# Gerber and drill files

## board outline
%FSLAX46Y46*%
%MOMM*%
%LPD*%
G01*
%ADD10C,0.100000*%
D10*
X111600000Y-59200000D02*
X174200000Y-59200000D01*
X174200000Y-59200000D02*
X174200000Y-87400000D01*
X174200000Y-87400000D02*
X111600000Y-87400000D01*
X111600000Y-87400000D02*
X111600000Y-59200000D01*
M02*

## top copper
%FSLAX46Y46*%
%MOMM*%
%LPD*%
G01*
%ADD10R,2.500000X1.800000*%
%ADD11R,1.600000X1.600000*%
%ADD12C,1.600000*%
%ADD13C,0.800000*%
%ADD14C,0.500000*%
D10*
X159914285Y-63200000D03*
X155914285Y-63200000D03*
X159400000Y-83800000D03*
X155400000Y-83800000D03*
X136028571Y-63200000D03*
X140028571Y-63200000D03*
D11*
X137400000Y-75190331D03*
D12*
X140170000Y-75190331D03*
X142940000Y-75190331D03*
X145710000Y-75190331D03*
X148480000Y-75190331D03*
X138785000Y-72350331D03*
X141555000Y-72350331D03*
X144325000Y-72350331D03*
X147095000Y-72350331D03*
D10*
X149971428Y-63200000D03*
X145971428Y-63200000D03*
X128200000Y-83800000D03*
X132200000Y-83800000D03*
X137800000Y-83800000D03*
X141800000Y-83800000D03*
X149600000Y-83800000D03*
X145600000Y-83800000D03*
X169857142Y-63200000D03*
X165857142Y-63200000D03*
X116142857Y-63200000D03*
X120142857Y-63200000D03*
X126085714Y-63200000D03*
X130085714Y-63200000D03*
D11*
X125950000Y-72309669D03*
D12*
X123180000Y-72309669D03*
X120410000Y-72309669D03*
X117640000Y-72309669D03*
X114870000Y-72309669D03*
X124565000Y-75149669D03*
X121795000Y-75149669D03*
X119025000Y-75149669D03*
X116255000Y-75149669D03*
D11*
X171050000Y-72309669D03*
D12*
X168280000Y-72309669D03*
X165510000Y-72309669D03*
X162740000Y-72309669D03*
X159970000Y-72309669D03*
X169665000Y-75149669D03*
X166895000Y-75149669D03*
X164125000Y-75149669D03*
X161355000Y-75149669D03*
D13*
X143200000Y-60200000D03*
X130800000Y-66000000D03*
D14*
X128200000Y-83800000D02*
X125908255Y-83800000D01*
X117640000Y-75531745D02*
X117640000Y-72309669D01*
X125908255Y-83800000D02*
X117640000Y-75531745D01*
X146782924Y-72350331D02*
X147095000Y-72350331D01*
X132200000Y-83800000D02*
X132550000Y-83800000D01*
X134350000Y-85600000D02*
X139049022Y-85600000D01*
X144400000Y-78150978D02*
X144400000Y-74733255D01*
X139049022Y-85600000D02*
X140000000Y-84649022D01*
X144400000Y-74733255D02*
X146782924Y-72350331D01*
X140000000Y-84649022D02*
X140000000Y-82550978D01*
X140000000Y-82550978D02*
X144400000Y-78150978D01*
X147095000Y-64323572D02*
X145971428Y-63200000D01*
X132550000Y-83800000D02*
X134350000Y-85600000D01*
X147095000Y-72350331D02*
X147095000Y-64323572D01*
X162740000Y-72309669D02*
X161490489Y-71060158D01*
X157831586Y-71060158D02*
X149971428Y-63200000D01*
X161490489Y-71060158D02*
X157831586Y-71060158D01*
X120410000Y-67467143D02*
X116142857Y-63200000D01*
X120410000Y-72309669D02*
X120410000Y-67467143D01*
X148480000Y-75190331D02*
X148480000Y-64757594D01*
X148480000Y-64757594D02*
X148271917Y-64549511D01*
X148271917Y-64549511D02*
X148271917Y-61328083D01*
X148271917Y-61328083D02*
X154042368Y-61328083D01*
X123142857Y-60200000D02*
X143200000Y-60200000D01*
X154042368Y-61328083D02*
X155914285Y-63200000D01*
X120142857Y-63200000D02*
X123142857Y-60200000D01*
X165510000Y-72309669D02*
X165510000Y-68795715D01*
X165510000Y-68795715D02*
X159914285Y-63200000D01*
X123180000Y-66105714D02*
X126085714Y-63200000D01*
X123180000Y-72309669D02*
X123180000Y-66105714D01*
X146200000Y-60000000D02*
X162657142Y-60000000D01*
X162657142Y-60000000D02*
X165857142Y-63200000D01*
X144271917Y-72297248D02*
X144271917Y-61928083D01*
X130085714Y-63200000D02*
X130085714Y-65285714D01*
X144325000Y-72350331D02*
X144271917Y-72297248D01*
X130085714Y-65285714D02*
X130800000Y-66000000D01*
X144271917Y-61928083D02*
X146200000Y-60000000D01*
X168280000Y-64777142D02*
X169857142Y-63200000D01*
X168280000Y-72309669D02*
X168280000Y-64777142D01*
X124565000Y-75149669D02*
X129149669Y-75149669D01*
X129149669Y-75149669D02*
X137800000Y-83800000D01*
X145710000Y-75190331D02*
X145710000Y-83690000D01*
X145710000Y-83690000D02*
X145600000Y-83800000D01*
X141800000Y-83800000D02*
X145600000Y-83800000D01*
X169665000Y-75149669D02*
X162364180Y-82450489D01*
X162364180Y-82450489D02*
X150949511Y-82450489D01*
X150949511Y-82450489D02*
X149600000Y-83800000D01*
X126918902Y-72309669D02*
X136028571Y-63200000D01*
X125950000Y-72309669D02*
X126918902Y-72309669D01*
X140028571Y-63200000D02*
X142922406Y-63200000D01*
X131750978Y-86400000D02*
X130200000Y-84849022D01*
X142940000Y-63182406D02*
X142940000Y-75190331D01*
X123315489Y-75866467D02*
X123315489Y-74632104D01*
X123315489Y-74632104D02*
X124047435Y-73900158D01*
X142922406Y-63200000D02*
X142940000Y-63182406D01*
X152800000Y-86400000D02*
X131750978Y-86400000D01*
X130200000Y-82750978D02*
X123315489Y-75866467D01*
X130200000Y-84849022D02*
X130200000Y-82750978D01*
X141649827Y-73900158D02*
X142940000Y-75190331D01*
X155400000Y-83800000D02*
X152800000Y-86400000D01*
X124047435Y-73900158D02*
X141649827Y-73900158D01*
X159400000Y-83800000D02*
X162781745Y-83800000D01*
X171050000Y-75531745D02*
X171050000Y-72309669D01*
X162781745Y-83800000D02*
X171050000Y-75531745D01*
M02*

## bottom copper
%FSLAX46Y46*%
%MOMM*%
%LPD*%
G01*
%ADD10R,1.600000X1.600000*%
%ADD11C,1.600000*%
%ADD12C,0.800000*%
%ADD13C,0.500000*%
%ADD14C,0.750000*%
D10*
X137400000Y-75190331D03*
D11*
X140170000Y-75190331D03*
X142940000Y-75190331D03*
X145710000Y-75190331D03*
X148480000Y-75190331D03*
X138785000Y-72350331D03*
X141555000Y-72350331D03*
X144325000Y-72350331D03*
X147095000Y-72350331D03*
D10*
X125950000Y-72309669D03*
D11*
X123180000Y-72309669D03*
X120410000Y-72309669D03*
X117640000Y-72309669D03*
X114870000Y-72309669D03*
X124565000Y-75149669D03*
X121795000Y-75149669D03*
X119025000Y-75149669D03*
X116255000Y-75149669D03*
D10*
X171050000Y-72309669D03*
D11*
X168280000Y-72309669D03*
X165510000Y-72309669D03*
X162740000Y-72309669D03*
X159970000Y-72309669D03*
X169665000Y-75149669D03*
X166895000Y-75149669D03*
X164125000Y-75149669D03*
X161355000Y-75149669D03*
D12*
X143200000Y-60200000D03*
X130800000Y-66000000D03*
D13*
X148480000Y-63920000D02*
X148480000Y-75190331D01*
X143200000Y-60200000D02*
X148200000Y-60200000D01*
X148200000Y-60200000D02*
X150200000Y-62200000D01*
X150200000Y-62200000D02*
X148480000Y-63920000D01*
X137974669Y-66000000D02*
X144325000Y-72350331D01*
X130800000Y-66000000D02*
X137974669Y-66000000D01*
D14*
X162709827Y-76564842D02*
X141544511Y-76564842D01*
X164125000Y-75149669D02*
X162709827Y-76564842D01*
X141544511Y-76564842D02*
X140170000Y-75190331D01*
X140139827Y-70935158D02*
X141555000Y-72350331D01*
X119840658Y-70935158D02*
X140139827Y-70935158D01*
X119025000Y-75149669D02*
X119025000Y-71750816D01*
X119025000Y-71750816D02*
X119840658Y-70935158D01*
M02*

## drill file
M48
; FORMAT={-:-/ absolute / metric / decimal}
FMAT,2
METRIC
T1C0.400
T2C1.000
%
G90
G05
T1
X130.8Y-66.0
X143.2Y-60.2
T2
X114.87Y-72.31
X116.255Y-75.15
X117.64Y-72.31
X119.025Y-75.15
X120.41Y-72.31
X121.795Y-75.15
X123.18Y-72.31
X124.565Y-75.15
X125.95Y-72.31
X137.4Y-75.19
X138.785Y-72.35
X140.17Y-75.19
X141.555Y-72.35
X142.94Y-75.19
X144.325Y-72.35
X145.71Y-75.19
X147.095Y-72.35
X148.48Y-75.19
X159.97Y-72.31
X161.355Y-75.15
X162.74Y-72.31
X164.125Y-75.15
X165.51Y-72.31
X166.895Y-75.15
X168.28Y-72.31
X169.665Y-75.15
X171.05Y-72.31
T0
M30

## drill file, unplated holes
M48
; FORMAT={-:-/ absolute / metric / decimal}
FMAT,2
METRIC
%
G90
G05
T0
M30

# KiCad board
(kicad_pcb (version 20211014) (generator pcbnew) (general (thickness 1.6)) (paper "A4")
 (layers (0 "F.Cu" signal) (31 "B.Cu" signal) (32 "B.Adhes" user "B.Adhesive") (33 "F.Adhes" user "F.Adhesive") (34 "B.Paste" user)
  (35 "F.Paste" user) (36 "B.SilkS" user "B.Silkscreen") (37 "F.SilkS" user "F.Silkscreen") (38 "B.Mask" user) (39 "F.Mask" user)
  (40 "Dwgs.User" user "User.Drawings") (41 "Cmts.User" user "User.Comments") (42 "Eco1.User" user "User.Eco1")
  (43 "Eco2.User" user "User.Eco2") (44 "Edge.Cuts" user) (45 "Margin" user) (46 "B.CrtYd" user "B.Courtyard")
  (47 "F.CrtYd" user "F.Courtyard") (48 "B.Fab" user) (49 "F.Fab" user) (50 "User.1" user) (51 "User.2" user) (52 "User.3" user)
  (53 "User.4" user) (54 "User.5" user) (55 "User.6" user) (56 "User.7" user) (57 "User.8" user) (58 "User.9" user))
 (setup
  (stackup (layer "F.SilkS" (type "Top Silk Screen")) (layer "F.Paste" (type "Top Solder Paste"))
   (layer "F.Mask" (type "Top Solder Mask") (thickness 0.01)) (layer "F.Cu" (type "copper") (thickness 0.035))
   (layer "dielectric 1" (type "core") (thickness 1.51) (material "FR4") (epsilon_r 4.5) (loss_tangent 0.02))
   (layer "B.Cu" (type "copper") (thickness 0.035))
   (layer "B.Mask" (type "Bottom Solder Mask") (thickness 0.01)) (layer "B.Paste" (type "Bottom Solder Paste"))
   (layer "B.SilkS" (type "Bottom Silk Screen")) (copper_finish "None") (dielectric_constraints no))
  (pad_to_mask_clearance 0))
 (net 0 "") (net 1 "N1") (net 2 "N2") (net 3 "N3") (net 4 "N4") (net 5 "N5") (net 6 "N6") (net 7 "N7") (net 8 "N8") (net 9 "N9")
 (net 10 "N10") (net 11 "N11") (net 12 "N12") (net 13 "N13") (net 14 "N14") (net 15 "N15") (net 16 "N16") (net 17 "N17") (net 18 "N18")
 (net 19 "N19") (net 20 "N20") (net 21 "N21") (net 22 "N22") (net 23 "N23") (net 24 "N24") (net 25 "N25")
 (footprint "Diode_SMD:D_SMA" (layer "F.Cu") (at 157.914285 63.2 180)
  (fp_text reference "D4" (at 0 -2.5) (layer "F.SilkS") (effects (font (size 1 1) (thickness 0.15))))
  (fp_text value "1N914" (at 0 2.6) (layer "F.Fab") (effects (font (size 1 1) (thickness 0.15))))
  (pad "1" smd rect (at -2 0 180) (size 2.5 1.8) (layers "F.Cu" "F.Paste" "F.Mask") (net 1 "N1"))
  (pad "2" smd rect (at 2 0 180) (size 2.5 1.8) (layers "F.Cu" "F.Paste" "F.Mask") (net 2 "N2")))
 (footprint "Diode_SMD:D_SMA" (layer "F.Cu") (at 157.4 83.8 180)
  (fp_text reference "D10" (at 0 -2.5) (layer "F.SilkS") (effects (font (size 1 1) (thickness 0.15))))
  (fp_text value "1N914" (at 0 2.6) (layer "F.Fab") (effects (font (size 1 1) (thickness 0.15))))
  (pad "1" smd rect (at -2 0 180) (size 2.5 1.8) (layers "F.Cu" "F.Paste" "F.Mask") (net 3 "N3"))
  (pad "2" smd rect (at 2 0 180) (size 2.5 1.8) (layers "F.Cu" "F.Paste" "F.Mask") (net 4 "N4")))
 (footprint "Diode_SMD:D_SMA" (layer "F.Cu") (at 138.028571 63.2)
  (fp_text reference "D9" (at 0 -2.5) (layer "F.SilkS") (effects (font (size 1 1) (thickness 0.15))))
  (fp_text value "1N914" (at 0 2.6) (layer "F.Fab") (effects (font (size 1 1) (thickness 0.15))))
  (pad "1" smd rect (at -2 0) (size 2.5 1.8) (layers "F.Cu" "F.Paste" "F.Mask") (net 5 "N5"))
  (pad "2" smd rect (at 2 0) (size 2.5 1.8) (layers "F.Cu" "F.Paste" "F.Mask") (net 4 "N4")))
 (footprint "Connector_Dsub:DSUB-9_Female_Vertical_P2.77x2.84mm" (layer "F.Cu") (at 137.4 75.190331 180)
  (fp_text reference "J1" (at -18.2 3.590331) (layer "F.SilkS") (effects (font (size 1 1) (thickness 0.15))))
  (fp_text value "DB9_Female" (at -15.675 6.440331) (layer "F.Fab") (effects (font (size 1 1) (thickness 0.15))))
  (pad "1" thru_hole rect (at 0 0 180) (size 1.6 1.6) (drill 1) (layers *.Cu *.Mask) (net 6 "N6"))
  (pad "2" thru_hole circle (at -2.77 0 180) (size 1.6 1.6) (drill 1) (layers *.Cu *.Mask) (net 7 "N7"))
  (pad "3" thru_hole circle (at -5.54 0 180) (size 1.6 1.6) (drill 1) (layers *.Cu *.Mask) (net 4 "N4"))
  (pad "4" thru_hole circle (at -8.31 0 180) (size 1.6 1.6) (drill 1) (layers *.Cu *.Mask) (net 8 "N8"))
  (pad "5" thru_hole circle (at -11.08 0 180) (size 1.6 1.6) (drill 1) (layers *.Cu *.Mask) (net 2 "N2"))
  (pad "6" thru_hole circle (at -1.385 2.84 180) (size 1.6 1.6) (drill 1) (layers *.Cu *.Mask) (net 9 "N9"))
  (pad "7" thru_hole circle (at -4.155 2.84 180) (size 1.6 1.6) (drill 1) (layers *.Cu *.Mask) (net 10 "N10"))
  (pad "8" thru_hole circle (at -6.925 2.84 180) (size 1.6 1.6) (drill 1) (layers *.Cu *.Mask) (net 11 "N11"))
  (pad "9" thru_hole circle (at -9.695 2.84 180) (size 1.6 1.6) (drill 1) (layers *.Cu *.Mask) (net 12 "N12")))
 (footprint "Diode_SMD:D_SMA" (layer "F.Cu") (at 147.971428 63.2 180)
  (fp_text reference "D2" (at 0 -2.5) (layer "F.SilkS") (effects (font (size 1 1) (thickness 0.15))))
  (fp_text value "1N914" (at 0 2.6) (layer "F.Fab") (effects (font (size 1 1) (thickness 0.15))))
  (pad "1" smd rect (at -2 0 180) (size 2.5 1.8) (layers "F.Cu" "F.Paste" "F.Mask") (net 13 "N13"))
  (pad "2" smd rect (at 2 0 180) (size 2.5 1.8) (layers "F.Cu" "F.Paste" "F.Mask") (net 12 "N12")))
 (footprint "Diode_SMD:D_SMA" (layer "F.Cu") (at 130.2 83.8)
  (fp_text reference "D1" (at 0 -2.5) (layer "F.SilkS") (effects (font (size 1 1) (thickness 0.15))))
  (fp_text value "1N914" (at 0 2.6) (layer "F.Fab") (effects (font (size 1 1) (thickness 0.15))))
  (pad "1" smd rect (at -2 0) (size 2.5 1.8) (layers "F.Cu" "F.Paste" "F.Mask") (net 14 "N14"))
  (pad "2" smd rect (at 2 0) (size 2.5 1.8) (layers "F.Cu" "F.Paste" "F.Mask") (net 12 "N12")))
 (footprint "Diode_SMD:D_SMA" (layer "F.Cu") (at 139.8 83.8)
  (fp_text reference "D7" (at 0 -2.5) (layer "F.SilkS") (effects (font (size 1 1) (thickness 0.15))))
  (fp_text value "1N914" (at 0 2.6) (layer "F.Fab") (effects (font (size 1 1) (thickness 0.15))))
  (pad "1" smd rect (at -2 0) (size 2.5 1.8) (layers "F.Cu" "F.Paste" "F.Mask") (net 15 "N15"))
  (pad "2" smd rect (at 2 0) (size 2.5 1.8) (layers "F.Cu" "F.Paste" "F.Mask") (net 8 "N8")))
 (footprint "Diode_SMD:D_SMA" (layer "F.Cu") (at 147.6 83.8 180)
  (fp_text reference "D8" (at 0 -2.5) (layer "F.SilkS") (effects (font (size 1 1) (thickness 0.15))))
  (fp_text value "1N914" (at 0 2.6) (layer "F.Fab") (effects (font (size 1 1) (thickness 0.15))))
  (pad "1" smd rect (at -2 0 180) (size 2.5 1.8) (layers "F.Cu" "F.Paste" "F.Mask") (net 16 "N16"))
  (pad "2" smd rect (at 2 0 180) (size 2.5 1.8) (layers "F.Cu" "F.Paste" "F.Mask") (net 8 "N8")))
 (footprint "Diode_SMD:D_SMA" (layer "F.Cu") (at 167.857142 63.2 180)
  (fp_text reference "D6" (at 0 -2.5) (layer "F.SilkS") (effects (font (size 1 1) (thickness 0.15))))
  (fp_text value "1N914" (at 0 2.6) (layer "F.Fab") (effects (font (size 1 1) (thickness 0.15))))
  (pad "1" smd rect (at -2 0 180) (size 2.5 1.8) (layers "F.Cu" "F.Paste" "F.Mask") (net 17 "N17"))
  (pad "2" smd rect (at 2 0 180) (size 2.5 1.8) (layers "F.Cu" "F.Paste" "F.Mask") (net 11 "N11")))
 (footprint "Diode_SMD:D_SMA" (layer "F.Cu") (at 118.142857 63.2)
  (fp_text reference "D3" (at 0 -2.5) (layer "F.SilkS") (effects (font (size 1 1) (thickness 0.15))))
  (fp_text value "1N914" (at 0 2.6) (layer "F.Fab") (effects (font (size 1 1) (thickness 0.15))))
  (pad "1" smd rect (at -2 0) (size 2.5 1.8) (layers "F.Cu" "F.Paste" "F.Mask") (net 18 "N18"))
  (pad "2" smd rect (at 2 0) (size 2.5 1.8) (layers "F.Cu" "F.Paste" "F.Mask") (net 2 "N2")))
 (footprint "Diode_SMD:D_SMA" (layer "F.Cu") (at 128.085714 63.2)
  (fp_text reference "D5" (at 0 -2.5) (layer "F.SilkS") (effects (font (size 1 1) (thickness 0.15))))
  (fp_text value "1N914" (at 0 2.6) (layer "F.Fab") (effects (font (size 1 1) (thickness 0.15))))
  (pad "1" smd rect (at -2 0) (size 2.5 1.8) (layers "F.Cu" "F.Paste" "F.Mask") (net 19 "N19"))
  (pad "2" smd rect (at 2 0) (size 2.5 1.8) (layers "F.Cu" "F.Paste" "F.Mask") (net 11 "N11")))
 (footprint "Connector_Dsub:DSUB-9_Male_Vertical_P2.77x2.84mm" (layer "B.Cu") (at 125.95 72.309669 180)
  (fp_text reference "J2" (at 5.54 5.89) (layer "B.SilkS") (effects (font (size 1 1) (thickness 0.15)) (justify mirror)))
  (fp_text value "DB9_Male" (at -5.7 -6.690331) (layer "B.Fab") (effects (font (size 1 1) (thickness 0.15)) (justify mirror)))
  (pad "1" thru_hole rect (at 0 0 180) (size 1.6 1.6) (drill 1) (layers *.Cu *.Mask) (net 5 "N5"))
  (pad "2" thru_hole circle (at 2.77 0 180) (size 1.6 1.6) (drill 1) (layers *.Cu *.Mask) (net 19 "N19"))
  (pad "3" thru_hole circle (at 5.54 0 180) (size 1.6 1.6) (drill 1) (layers *.Cu *.Mask) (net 18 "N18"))
  (pad "4" thru_hole circle (at 8.31 0 180) (size 1.6 1.6) (drill 1) (layers *.Cu *.Mask) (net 14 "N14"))
  (pad "5" thru_hole circle (at 11.08 0 180) (size 1.6 1.6) (drill 1) (layers *.Cu *.Mask) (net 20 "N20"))
  (pad "6" thru_hole circle (at 1.385 -2.84 180) (size 1.6 1.6) (drill 1) (layers *.Cu *.Mask) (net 15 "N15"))
  (pad "7" thru_hole circle (at 4.155 -2.84 180) (size 1.6 1.6) (drill 1) (layers *.Cu *.Mask) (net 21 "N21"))
  (pad "8" thru_hole circle (at 6.925 -2.84 180) (size 1.6 1.6) (drill 1) (layers *.Cu *.Mask) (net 10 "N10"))
  (pad "9" thru_hole circle (at 9.695 -2.84 180) (size 1.6 1.6) (drill 1) (layers *.Cu *.Mask) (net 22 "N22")))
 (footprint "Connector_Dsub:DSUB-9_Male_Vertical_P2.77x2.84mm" (layer "B.Cu") (at 171.05 72.309669 180)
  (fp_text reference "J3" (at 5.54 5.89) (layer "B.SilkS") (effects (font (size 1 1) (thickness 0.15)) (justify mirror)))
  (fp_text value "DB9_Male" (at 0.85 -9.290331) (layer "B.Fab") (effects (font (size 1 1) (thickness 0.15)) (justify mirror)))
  (pad "1" thru_hole rect (at 0 0 180) (size 1.6 1.6) (drill 1) (layers *.Cu *.Mask) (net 3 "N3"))
  (pad "2" thru_hole circle (at 2.77 0 180) (size 1.6 1.6) (drill 1) (layers *.Cu *.Mask) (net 17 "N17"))
  (pad "3" thru_hole circle (at 5.54 0 180) (size 1.6 1.6) (drill 1) (layers *.Cu *.Mask) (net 1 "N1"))
  (pad "4" thru_hole circle (at 8.31 0 180) (size 1.6 1.6) (drill 1) (layers *.Cu *.Mask) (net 13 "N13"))
  (pad "5" thru_hole circle (at 11.08 0 180) (size 1.6 1.6) (drill 1) (layers *.Cu *.Mask) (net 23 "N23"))
  (pad "6" thru_hole circle (at 1.385 -2.84 180) (size 1.6 1.6) (drill 1) (layers *.Cu *.Mask) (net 16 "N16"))
  (pad "7" thru_hole circle (at 4.155 -2.84 180) (size 1.6 1.6) (drill 1) (layers *.Cu *.Mask) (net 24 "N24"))
  (pad "8" thru_hole circle (at 6.925 -2.84 180) (size 1.6 1.6) (drill 1) (layers *.Cu *.Mask) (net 7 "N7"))
  (pad "9" thru_hole circle (at 9.695 -2.84 180) (size 1.6 1.6) (drill 1) (layers *.Cu *.Mask) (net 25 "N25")))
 (gr_rect (start 111.6 59.2) (end 174.2 87.4) (layer "Edge.Cuts") (width 0.1) (fill none))
 (segment (start 128.2 83.8) (end 125.908255 83.8) (width 0.5) (layer "F.Cu") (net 14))
 (segment (start 117.64 75.531745) (end 117.64 72.309669) (width 0.5) (layer "F.Cu") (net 14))
 (segment (start 125.908255 83.8) (end 117.64 75.531745) (width 0.5) (layer "F.Cu") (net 14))
 (segment (start 146.782924 72.350331) (end 147.095 72.350331) (width 0.5) (layer "F.Cu") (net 12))
 (segment (start 132.2 83.8) (end 132.55 83.8) (width 0.5) (layer "F.Cu") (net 12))
 (segment (start 134.35 85.6) (end 139.049022 85.6) (width 0.5) (layer "F.Cu") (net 12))
 (segment (start 144.4 78.150978) (end 144.4 74.733255) (width 0.5) (layer "F.Cu") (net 12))
 (segment (start 139.049022 85.6) (end 140 84.649022) (width 0.5) (layer "F.Cu") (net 12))
 (segment (start 144.4 74.733255) (end 146.782924 72.350331) (width 0.5) (layer "F.Cu") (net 12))
 (segment (start 140 84.649022) (end 140 82.550978) (width 0.5) (layer "F.Cu") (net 12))
 (segment (start 140 82.550978) (end 144.4 78.150978) (width 0.5) (layer "F.Cu") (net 12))
 (segment (start 147.095 64.323572) (end 145.971428 63.2) (width 0.5) (layer "F.Cu") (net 12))
 (segment (start 132.55 83.8) (end 134.35 85.6) (width 0.5) (layer "F.Cu") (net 12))
 (segment (start 147.095 72.350331) (end 147.095 64.323572) (width 0.5) (layer "F.Cu") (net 12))
 (segment (start 162.74 72.309669) (end 161.490489 71.060158) (width 0.5) (layer "F.Cu") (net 13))
 (segment (start 157.831586 71.060158) (end 149.971428 63.2) (width 0.5) (layer "F.Cu") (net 13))
 (segment (start 161.490489 71.060158) (end 157.831586 71.060158) (width 0.5) (layer "F.Cu") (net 13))
 (segment (start 120.41 67.467143) (end 116.142857 63.2) (width 0.5) (layer "F.Cu") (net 18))
 (segment (start 120.41 72.309669) (end 120.41 67.467143) (width 0.5) (layer "F.Cu") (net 18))
 (segment (start 148.48 75.190331) (end 148.48 64.757594) (width 0.5) (layer "F.Cu") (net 2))
 (segment (start 148.48 64.757594) (end 148.271917 64.549511) (width 0.5) (layer "F.Cu") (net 2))
 (segment (start 148.271917 64.549511) (end 148.271917 61.328083) (width 0.5) (layer "F.Cu") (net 2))
 (segment (start 148.271917 61.328083) (end 154.042368 61.328083) (width 0.5) (layer "F.Cu") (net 2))
 (segment (start 123.142857 60.2) (end 143.2 60.2) (width 0.5) (layer "F.Cu") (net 2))
 (segment (start 154.042368 61.328083) (end 155.914285 63.2) (width 0.5) (layer "F.Cu") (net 2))
 (segment (start 120.142857 63.2) (end 123.142857 60.2) (width 0.5) (layer "F.Cu") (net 2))
 (via (at 143.2 60.2) (size 0.8) (drill 0.4) (layers "F.Cu" "B.Cu") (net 2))
 (segment (start 148.48 63.92) (end 148.48 75.190331) (width 0.5) (layer "B.Cu") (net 2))
 (segment (start 143.2 60.2) (end 148.2 60.2) (width 0.5) (layer "B.Cu") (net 2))
 (segment (start 148.2 60.2) (end 150.2 62.2) (width 0.5) (layer "B.Cu") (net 2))
 (segment (start 150.2 62.2) (end 148.48 63.92) (width 0.5) (layer "B.Cu") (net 2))
 (segment (start 165.51 72.309669) (end 165.51 68.795715) (width 0.5) (layer "F.Cu") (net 1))
 (segment (start 165.51 68.795715) (end 159.914285 63.2) (width 0.5) (layer "F.Cu") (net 1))
 (segment (start 123.18 66.105714) (end 126.085714 63.2) (width 0.5) (layer "F.Cu") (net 19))
 (segment (start 123.18 72.309669) (end 123.18 66.105714) (width 0.5) (layer "F.Cu") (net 19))
 (segment (start 146.2 60) (end 162.657142 60) (width 0.5) (layer "F.Cu") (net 11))
 (segment (start 162.657142 60) (end 165.857142 63.2) (width 0.5) (layer "F.Cu") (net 11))
 (segment (start 144.271917 72.297248) (end 144.271917 61.928083) (width 0.5) (layer "F.Cu") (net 11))
 (segment (start 130.085714 63.2) (end 130.085714 65.285714) (width 0.5) (layer "F.Cu") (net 11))
 (segment (start 144.325 72.350331) (end 144.271917 72.297248) (width 0.5) (layer "F.Cu") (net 11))
 (segment (start 130.085714 65.285714) (end 130.8 66) (width 0.5) (layer "F.Cu") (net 11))
 (segment (start 144.271917 61.928083) (end 146.2 60) (width 0.5) (layer "F.Cu") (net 11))
 (via (at 130.8 66) (size 0.8) (drill 0.4) (layers "F.Cu" "B.Cu") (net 11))
 (segment (start 137.974669 66) (end 144.325 72.350331) (width 0.5) (layer "B.Cu") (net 11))
 (segment (start 130.8 66) (end 137.974669 66) (width 0.5) (layer "B.Cu") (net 11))
 (segment (start 168.28 64.777142) (end 169.857142 63.2) (width 0.5) (layer "F.Cu") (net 17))
 (segment (start 168.28 72.309669) (end 168.28 64.777142) (width 0.5) (layer "F.Cu") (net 17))
 (segment (start 124.565 75.149669) (end 129.149669 75.149669) (width 0.5) (layer "F.Cu") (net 15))
 (segment (start 129.149669 75.149669) (end 137.8 83.8) (width 0.5) (layer "F.Cu") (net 15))
 (segment (start 145.71 75.190331) (end 145.71 83.69) (width 0.5) (layer "F.Cu") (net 8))
 (segment (start 145.71 83.69) (end 145.6 83.8) (width 0.5) (layer "F.Cu") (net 8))
 (segment (start 141.8 83.8) (end 145.6 83.8) (width 0.5) (layer "F.Cu") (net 8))
 (segment (start 169.665 75.149669) (end 162.36418 82.450489) (width 0.5) (layer "F.Cu") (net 16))
 (segment (start 162.36418 82.450489) (end 150.949511 82.450489) (width 0.5) (layer "F.Cu") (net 16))
 (segment (start 150.949511 82.450489) (end 149.6 83.8) (width 0.5) (layer "F.Cu") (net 16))
 (segment (start 126.918902 72.309669) (end 136.028571 63.2) (width 0.5) (layer "F.Cu") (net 5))
 (segment (start 125.95 72.309669) (end 126.918902 72.309669) (width 0.5) (layer "F.Cu") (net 5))
 (segment (start 140.028571 63.2) (end 142.922406 63.2) (width 0.5) (layer "F.Cu") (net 4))
 (segment (start 131.750978 86.4) (end 130.2 84.849022) (width 0.5) (layer "F.Cu") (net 4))
 (segment (start 142.94 63.182406) (end 142.94 75.190331) (width 0.5) (layer "F.Cu") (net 4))
 (segment (start 123.315489 75.866467) (end 123.315489 74.632104) (width 0.5) (layer "F.Cu") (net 4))
 (segment (start 123.315489 74.632104) (end 124.047435 73.900158) (width 0.5) (layer "F.Cu") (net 4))
 (segment (start 142.922406 63.2) (end 142.94 63.182406) (width 0.5) (layer "F.Cu") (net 4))
 (segment (start 152.8 86.4) (end 131.750978 86.4) (width 0.5) (layer "F.Cu") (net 4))
 (segment (start 130.2 82.750978) (end 123.315489 75.866467) (width 0.5) (layer "F.Cu") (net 4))
 (segment (start 130.2 84.849022) (end 130.2 82.750978) (width 0.5) (layer "F.Cu") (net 4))
 (segment (start 141.649827 73.900158) (end 142.94 75.190331) (width 0.5) (layer "F.Cu") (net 4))
 (segment (start 155.4 83.8) (end 152.8 86.4) (width 0.5) (layer "F.Cu") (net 4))
 (segment (start 124.047435 73.900158) (end 141.649827 73.900158) (width 0.5) (layer "F.Cu") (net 4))
 (segment (start 159.4 83.8) (end 162.781745 83.8) (width 0.5) (layer "F.Cu") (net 3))
 (segment (start 171.05 75.531745) (end 171.05 72.309669) (width 0.5) (layer "F.Cu") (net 3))
 (segment (start 162.781745 83.8) (end 171.05 75.531745) (width 0.5) (layer "F.Cu") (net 3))
 (segment (start 162.709827 76.564842) (end 141.544511 76.564842) (width 0.75) (layer "B.Cu") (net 7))
 (segment (start 164.125 75.149669) (end 162.709827 76.564842) (width 0.75) (layer "B.Cu") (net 7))
 (segment (start 141.544511 76.564842) (end 140.17 75.190331) (width 0.75) (layer "B.Cu") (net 7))
 (segment (start 140.139827 70.935158) (end 141.555 72.350331) (width 0.75) (layer "B.Cu") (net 10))
 (segment (start 119.840658 70.935158) (end 140.139827 70.935158) (width 0.75) (layer "B.Cu") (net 10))
 (segment (start 119.025 75.149669) (end 119.025 71.750816) (width 0.75) (layer "B.Cu") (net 10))
 (segment (start 119.025 71.750816) (end 119.840658 70.935158) (width 0.75) (layer "B.Cu") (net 10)))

